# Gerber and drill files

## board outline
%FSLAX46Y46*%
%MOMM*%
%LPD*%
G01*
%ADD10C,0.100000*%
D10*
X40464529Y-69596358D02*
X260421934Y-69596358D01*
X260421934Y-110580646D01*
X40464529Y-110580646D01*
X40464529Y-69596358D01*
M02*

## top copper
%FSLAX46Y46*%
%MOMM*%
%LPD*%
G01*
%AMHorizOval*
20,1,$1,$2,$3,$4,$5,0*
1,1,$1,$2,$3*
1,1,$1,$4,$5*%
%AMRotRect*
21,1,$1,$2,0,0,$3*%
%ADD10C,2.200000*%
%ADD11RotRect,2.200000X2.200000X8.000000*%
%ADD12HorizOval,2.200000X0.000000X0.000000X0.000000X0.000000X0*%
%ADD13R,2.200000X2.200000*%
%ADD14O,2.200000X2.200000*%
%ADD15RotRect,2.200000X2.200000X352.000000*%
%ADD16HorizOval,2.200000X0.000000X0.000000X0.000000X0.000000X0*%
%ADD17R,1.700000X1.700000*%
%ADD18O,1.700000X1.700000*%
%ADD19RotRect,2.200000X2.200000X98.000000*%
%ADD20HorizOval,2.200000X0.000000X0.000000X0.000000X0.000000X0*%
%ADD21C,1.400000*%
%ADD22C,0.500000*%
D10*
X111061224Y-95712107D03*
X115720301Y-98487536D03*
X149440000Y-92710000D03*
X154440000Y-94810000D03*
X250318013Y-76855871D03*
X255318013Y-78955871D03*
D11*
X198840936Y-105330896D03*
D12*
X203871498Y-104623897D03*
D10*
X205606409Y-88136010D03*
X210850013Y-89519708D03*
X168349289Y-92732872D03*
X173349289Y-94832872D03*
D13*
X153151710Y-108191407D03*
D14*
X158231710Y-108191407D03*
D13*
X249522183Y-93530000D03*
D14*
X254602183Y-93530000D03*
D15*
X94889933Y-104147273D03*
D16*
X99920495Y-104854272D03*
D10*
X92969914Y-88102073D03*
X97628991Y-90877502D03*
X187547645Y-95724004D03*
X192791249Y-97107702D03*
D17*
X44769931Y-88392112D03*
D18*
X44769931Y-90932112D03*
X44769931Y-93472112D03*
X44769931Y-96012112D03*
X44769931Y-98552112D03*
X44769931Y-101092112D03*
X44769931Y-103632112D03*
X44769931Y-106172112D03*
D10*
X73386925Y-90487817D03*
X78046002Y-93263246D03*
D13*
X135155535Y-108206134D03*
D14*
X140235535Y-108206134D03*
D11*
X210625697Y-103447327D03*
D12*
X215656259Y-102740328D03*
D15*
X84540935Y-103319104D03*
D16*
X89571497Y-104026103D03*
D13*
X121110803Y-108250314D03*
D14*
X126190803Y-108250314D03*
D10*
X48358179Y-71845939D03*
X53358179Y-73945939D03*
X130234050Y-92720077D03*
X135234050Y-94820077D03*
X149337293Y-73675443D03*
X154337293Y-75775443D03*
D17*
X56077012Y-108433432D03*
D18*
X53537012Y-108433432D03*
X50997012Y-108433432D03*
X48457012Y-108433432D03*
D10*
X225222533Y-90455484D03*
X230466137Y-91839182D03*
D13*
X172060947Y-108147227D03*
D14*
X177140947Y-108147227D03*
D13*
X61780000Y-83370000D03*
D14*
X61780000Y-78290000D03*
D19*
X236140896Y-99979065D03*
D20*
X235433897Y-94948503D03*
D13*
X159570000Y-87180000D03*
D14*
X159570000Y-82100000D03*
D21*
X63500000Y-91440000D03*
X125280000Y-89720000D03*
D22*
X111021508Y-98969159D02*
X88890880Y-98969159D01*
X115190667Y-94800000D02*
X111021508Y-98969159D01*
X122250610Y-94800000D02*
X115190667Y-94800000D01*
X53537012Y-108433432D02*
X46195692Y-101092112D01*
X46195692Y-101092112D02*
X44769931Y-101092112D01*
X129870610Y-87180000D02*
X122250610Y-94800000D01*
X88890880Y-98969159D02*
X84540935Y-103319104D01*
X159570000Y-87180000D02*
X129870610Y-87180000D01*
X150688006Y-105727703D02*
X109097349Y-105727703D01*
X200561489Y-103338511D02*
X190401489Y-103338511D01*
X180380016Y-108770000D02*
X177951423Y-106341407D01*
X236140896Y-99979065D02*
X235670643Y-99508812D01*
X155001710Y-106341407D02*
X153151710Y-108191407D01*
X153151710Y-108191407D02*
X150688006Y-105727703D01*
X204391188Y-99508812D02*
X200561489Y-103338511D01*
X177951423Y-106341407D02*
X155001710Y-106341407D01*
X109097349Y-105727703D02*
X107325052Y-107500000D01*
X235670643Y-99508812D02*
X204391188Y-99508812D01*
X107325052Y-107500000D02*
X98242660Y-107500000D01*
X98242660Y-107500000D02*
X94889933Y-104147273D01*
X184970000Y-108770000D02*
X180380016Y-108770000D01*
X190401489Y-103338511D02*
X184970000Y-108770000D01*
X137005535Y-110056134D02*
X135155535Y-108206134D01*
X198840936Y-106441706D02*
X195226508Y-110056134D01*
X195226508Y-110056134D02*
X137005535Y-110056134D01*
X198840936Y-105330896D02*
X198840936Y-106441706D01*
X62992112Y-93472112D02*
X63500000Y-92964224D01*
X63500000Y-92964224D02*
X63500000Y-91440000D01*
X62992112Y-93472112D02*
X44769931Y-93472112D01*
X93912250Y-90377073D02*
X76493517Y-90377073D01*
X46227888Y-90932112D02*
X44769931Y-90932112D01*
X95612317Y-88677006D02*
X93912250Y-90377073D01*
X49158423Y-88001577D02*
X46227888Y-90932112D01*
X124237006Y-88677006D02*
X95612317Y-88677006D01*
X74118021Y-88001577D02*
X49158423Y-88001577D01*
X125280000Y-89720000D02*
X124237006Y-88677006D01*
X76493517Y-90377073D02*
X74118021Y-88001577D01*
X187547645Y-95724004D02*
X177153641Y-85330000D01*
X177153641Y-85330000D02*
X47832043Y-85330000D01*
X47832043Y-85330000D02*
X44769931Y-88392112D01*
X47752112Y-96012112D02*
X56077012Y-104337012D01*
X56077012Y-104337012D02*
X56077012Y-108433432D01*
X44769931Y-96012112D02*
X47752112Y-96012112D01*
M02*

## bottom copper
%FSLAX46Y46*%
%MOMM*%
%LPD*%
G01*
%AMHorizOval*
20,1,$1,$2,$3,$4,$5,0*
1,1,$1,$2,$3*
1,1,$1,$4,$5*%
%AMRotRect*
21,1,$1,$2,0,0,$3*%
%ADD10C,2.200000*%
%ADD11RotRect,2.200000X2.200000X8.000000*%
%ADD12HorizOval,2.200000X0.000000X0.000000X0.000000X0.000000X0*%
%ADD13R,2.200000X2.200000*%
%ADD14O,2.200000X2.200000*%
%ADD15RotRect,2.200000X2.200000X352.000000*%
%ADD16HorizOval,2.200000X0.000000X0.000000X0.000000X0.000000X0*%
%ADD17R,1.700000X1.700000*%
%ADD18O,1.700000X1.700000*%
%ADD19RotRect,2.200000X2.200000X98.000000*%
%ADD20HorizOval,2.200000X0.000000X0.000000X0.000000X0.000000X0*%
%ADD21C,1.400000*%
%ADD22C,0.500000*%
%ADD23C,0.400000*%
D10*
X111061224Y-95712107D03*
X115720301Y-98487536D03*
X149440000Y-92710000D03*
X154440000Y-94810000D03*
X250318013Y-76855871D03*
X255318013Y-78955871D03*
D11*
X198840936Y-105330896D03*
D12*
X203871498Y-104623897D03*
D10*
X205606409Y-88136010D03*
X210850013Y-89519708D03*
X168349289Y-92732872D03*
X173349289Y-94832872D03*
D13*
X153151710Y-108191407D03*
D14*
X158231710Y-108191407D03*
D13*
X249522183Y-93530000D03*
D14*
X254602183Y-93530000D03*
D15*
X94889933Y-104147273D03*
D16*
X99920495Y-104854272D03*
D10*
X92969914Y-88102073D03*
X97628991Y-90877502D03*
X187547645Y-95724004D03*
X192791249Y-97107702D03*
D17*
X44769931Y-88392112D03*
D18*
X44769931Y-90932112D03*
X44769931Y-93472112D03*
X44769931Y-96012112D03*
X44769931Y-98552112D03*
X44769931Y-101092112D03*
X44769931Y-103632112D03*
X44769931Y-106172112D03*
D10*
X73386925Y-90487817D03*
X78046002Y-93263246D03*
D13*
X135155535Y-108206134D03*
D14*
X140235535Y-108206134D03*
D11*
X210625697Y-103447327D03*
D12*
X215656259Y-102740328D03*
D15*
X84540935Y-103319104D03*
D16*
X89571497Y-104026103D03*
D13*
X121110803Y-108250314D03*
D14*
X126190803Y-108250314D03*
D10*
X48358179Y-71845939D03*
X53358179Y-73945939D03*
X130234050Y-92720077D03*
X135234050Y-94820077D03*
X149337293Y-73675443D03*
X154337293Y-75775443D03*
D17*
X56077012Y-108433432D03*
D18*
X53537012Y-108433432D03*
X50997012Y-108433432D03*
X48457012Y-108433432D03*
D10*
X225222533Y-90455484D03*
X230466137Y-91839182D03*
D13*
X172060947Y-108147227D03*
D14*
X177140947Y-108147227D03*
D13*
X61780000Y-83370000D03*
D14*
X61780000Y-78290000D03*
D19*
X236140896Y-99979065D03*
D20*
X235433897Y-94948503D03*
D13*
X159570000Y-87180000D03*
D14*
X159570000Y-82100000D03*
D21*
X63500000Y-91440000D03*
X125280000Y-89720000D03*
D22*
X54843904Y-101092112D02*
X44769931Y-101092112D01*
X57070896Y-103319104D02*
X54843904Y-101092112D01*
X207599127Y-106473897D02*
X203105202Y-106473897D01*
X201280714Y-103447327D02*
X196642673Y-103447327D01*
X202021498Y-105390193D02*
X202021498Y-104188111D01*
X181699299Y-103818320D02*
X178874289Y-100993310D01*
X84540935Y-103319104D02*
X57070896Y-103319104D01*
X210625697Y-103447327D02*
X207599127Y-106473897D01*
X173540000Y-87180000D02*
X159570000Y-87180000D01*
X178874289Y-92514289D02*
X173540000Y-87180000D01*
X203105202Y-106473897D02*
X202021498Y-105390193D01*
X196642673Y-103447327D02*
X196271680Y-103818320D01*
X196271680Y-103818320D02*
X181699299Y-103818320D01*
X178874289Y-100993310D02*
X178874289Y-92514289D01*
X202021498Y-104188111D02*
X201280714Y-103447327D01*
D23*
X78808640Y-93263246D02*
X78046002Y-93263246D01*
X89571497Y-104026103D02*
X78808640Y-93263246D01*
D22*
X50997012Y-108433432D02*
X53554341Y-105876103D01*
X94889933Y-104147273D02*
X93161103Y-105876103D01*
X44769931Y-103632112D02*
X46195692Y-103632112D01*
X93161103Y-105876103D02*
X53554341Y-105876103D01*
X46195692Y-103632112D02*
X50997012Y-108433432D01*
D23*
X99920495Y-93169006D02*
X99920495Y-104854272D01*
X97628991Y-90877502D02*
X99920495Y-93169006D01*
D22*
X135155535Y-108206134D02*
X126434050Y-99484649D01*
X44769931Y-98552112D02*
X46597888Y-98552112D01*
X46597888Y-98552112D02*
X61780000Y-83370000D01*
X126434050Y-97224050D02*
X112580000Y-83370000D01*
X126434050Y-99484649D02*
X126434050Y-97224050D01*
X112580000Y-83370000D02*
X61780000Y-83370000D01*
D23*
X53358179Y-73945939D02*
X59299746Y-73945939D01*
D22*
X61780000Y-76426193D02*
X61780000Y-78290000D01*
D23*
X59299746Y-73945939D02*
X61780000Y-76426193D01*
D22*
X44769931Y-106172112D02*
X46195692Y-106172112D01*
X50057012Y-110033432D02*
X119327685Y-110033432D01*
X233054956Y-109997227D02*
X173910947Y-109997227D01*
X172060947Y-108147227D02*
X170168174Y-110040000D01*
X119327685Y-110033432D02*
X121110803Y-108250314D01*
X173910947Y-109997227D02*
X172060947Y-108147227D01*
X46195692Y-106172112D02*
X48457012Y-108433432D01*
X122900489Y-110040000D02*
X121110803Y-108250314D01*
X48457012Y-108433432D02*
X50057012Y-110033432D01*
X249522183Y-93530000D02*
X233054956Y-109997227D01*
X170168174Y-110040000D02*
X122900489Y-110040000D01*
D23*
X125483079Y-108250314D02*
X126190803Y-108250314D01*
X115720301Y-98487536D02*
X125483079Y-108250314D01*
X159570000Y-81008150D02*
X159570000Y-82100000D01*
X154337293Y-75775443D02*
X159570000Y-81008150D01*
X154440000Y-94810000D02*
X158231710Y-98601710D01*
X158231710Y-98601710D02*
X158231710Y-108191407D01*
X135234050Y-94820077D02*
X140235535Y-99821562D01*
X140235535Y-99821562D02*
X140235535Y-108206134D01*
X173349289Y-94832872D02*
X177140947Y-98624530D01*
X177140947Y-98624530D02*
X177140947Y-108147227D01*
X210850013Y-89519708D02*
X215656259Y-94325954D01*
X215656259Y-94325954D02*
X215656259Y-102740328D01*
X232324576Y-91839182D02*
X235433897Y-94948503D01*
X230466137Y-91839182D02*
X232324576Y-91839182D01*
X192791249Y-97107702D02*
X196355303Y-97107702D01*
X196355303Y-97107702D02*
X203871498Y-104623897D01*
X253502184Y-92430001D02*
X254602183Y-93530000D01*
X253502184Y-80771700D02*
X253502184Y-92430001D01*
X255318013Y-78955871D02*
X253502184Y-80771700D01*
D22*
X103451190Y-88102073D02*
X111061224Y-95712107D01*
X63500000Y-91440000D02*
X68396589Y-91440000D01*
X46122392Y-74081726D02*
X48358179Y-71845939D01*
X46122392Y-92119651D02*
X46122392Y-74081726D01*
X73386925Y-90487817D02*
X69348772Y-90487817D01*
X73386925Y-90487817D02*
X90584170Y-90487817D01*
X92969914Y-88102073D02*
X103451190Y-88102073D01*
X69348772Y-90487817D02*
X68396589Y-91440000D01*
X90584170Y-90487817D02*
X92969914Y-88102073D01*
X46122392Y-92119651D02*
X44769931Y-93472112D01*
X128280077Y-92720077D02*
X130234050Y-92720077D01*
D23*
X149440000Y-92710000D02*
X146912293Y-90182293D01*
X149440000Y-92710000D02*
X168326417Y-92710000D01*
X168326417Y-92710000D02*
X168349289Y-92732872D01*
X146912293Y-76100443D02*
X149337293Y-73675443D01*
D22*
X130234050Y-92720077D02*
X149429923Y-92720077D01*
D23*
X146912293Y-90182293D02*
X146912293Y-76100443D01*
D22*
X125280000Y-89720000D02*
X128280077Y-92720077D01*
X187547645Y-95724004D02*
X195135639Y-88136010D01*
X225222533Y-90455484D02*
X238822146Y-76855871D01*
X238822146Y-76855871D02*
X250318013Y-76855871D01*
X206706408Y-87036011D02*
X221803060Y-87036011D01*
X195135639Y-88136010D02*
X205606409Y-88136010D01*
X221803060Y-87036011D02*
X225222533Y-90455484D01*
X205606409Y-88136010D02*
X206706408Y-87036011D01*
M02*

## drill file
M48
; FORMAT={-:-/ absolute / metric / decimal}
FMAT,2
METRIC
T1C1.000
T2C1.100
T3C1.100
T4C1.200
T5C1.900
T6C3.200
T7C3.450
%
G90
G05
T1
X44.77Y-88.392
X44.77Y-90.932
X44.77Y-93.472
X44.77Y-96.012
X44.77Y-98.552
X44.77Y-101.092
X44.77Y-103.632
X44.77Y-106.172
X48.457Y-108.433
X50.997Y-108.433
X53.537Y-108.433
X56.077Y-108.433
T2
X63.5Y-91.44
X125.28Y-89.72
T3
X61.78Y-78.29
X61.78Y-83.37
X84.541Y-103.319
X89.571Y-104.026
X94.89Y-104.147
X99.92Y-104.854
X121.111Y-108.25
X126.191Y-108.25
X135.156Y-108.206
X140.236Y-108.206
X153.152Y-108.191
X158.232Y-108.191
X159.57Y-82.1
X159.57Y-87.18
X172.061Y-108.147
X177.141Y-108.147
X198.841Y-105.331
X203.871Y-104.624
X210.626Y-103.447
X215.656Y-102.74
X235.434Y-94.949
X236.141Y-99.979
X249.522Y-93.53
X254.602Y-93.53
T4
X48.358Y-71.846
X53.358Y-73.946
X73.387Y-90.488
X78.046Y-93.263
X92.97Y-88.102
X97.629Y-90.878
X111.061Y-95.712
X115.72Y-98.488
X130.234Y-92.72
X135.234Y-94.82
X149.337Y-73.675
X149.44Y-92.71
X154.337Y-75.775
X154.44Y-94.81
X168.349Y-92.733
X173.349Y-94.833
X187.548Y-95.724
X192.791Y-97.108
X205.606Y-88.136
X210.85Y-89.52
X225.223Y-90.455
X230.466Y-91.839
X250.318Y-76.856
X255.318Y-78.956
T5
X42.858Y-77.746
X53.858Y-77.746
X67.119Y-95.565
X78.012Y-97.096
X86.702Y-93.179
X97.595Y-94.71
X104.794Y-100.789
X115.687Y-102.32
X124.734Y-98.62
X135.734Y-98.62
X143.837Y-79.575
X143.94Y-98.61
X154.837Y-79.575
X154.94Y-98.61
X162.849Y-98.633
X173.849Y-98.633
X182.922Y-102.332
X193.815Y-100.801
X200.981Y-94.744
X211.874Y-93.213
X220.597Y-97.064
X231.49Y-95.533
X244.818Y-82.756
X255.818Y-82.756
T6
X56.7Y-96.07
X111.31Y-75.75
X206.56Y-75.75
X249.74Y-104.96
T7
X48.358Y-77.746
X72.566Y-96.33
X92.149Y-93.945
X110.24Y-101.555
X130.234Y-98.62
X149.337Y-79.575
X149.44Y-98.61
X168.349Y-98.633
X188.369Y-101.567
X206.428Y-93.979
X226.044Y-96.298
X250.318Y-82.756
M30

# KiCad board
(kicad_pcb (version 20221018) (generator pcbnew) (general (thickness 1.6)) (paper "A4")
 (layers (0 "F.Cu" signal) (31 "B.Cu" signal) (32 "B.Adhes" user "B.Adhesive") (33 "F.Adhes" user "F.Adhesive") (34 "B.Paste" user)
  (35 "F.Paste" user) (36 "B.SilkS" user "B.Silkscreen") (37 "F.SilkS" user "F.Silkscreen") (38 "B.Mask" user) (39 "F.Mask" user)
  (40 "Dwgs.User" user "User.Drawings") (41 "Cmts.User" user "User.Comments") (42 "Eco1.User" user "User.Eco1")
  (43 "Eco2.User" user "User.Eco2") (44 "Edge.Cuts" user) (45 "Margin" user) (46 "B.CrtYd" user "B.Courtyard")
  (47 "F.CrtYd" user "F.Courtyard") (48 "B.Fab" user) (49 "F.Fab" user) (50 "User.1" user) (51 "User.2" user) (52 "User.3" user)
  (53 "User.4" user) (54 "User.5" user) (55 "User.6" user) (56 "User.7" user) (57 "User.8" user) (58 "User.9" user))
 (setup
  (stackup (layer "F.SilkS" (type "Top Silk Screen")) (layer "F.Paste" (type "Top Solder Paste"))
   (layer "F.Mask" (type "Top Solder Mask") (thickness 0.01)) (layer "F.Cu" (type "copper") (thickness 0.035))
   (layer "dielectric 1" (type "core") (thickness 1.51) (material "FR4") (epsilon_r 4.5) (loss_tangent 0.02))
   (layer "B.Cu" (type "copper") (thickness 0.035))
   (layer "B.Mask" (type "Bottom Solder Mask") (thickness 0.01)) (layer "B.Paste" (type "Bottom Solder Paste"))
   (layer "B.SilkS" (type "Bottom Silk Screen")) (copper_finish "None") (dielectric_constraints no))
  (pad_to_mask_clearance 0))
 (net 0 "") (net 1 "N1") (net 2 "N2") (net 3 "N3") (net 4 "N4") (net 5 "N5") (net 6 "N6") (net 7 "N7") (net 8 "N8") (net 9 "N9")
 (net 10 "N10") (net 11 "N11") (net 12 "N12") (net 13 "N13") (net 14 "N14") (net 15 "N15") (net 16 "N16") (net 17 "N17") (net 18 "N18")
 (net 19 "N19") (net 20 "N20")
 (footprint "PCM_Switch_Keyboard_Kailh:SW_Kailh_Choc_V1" (layer "F.Cu") (at 110.240103 101.554689 -8)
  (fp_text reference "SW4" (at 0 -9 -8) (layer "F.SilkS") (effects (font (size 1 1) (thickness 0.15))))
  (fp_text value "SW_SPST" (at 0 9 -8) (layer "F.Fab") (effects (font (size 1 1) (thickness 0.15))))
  (pad "" np_thru_hole circle (at -5.5 0 352) (size 1.9 1.9) (drill 1.9) (layers "*.Cu" "*.Mask"))
  (pad "" smd circle (at 0 -5.9 352) (size 1.25 1.25) (layers "F.Mask"))
  (pad "" np_thru_hole circle (at 0 0 352) (size 3.45 3.45) (drill 3.45) (layers "*.Cu" "*.Mask"))
  (pad "" smd circle (at 5 -3.8 352) (size 1.25 1.25) (layers "F.Mask"))
  (pad "" np_thru_hole circle (at 5.5 0 352) (size 1.9 1.9) (drill 1.9) (layers "*.Cu" "*.Mask"))
  (pad "1" thru_hole circle (at 0 -5.9 352) (size 2.2 2.2) (drill 1.2) (layers "*.Cu" "B.Mask") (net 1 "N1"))
  (pad "2" thru_hole circle (at 5 -3.8 352) (size 2.2 2.2) (drill 1.2) (layers "*.Cu" "B.Mask") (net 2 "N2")))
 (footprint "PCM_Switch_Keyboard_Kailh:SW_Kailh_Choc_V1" (layer "F.Cu") (at 149.44 98.61)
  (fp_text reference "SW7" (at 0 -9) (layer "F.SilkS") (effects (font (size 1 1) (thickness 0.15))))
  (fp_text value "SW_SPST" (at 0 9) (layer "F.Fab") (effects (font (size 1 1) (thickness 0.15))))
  (pad "" np_thru_hole circle (at -5.5 0) (size 1.9 1.9) (drill 1.9) (layers "*.Cu" "*.Mask"))
  (pad "" smd circle (at 0 -5.9) (size 1.25 1.25) (layers "F.Mask"))
  (pad "" np_thru_hole circle (at 0 0) (size 3.45 3.45) (drill 3.45) (layers "*.Cu" "*.Mask"))
  (pad "" smd circle (at 5 -3.8) (size 1.25 1.25) (layers "F.Mask"))
  (pad "" np_thru_hole circle (at 5.5 0) (size 1.9 1.9) (drill 1.9) (layers "*.Cu" "*.Mask"))
  (pad "1" thru_hole circle (at 0 -5.9) (size 2.2 2.2) (drill 1.2) (layers "*.Cu" "B.Mask") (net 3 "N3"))
  (pad "2" thru_hole circle (at 5 -3.8) (size 2.2 2.2) (drill 1.2) (layers "*.Cu" "B.Mask") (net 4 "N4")))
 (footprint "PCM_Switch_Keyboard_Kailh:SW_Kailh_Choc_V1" (layer "F.Cu") (at 250.318013 82.755871)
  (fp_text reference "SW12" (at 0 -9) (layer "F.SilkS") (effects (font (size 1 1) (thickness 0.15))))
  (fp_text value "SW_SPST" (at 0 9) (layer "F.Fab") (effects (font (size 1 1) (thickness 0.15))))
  (pad "" np_thru_hole circle (at -5.5 0) (size 1.9 1.9) (drill 1.9) (layers "*.Cu" "*.Mask"))
  (pad "" smd circle (at 0 -5.9) (size 1.25 1.25) (layers "F.Mask"))
  (pad "" np_thru_hole circle (at 0 0) (size 3.45 3.45) (drill 3.45) (layers "*.Cu" "*.Mask"))
  (pad "" smd circle (at 5 -3.8) (size 1.25 1.25) (layers "F.Mask"))
  (pad "" np_thru_hole circle (at 5.5 0) (size 1.9 1.9) (drill 1.9) (layers "*.Cu" "*.Mask"))
  (pad "1" thru_hole circle (at 0 -5.9) (size 2.2 2.2) (drill 1.2) (layers "*.Cu" "B.Mask") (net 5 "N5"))
  (pad "2" thru_hole circle (at 5 -3.8) (size 2.2 2.2) (drill 1.2) (layers "*.Cu" "B.Mask") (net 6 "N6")))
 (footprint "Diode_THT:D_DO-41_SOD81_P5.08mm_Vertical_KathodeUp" (layer "F.Cu") (at 198.840936 105.330896 8)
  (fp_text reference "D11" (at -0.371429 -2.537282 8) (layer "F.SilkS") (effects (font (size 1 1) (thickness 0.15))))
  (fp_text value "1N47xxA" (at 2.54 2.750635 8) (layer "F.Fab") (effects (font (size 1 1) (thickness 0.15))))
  (pad "1" thru_hole rect (at 0 0 8) (size 2.2 2.2) (drill 1.1) (layers "*.Cu" "*.Mask") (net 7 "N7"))
  (pad "2" thru_hole oval (at 5.08 0 8) (size 2.2 2.2) (drill 1.1) (layers "*.Cu" "*.Mask") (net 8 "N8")))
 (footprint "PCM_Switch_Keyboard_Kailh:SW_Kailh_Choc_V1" (layer "F.Cu") (at 206.42753 93.978592 8)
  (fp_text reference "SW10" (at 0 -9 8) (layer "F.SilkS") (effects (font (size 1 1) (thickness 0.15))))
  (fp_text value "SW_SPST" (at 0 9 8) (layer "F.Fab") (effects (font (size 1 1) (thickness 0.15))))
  (pad "" np_thru_hole circle (at -5.5 0 8) (size 1.9 1.9) (drill 1.9) (layers "*.Cu" "*.Mask"))
  (pad "" smd circle (at 0 -5.9 8) (size 1.25 1.25) (layers "F.Mask"))
  (pad "" np_thru_hole circle (at 0 0 8) (size 3.45 3.45) (drill 3.45) (layers "*.Cu" "*.Mask"))
  (pad "" smd circle (at 5 -3.8 8) (size 1.25 1.25) (layers "F.Mask"))
  (pad "" np_thru_hole circle (at 5.5 0 8) (size 1.9 1.9) (drill 1.9) (layers "*.Cu" "*.Mask"))
  (pad "1" thru_hole circle (at 0 -5.9 8) (size 2.2 2.2) (drill 1.2) (layers "*.Cu" "B.Mask") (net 5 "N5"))
  (pad "2" thru_hole circle (at 5 -3.8 8) (size 2.2 2.2) (drill 1.2) (layers "*.Cu" "B.Mask") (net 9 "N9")))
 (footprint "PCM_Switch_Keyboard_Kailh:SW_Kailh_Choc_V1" (layer "F.Cu") (at 168.349289 98.632872)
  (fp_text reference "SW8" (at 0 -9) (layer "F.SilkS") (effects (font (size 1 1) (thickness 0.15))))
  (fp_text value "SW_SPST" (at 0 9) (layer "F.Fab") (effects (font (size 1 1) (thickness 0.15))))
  (pad "" np_thru_hole circle (at -5.5 0) (size 1.9 1.9) (drill 1.9) (layers "*.Cu" "*.Mask"))
  (pad "" smd circle (at 0 -5.9) (size 1.25 1.25) (layers "F.Mask"))
  (pad "" np_thru_hole circle (at 0 0) (size 3.45 3.45) (drill 3.45) (layers "*.Cu" "*.Mask"))
  (pad "" smd circle (at 5 -3.8) (size 1.25 1.25) (layers "F.Mask"))
  (pad "" np_thru_hole circle (at 5.5 0) (size 1.9 1.9) (drill 1.9) (layers "*.Cu" "*.Mask"))
  (pad "1" thru_hole circle (at 0 -5.9) (size 2.2 2.2) (drill 1.2) (layers "*.Cu" "B.Mask") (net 3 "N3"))
  (pad "2" thru_hole circle (at 5 -3.8) (size 2.2 2.2) (drill 1.2) (layers "*.Cu" "B.Mask") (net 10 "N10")))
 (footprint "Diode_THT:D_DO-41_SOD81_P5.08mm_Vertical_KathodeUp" (layer "F.Cu") (at 153.15171 108.191407)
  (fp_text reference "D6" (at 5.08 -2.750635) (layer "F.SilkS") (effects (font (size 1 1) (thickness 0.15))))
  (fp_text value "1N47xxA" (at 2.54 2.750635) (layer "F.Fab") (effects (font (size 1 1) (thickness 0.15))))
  (pad "1" thru_hole rect (at 0 0) (size 2.2 2.2) (drill 1.1) (layers "*.Cu" "*.Mask") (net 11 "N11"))
  (pad "2" thru_hole oval (at 5.08 0) (size 2.2 2.2) (drill 1.1) (layers "*.Cu" "*.Mask") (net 4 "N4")))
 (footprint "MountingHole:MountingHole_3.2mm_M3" (layer "F.Cu") (at 249.74 104.96)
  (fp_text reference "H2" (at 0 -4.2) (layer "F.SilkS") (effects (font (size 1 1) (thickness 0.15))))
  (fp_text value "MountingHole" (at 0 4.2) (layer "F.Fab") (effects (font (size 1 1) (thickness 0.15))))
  (pad "" np_thru_hole circle (at 0 0) (size 3.2 3.2) (drill 3.2) (layers "*.Cu" "*.Mask")))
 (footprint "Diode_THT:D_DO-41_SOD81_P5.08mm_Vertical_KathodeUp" (layer "F.Cu") (at 249.522183 93.53)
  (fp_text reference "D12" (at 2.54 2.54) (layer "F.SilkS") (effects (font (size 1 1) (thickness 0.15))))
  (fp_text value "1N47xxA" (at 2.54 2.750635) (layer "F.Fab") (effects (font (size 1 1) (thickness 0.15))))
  (pad "1" thru_hole rect (at 0 0) (size 2.2 2.2) (drill 1.1) (layers "*.Cu" "*.Mask") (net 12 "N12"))
  (pad "2" thru_hole oval (at 5.08 0) (size 2.2 2.2) (drill 1.1) (layers "*.Cu" "*.Mask") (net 6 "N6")))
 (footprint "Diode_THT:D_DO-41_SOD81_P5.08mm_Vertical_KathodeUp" (layer "F.Cu") (at 94.889933 104.147273 -8)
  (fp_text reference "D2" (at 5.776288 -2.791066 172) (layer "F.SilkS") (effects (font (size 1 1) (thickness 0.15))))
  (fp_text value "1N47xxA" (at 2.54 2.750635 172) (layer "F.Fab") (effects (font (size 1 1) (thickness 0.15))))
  (pad "1" thru_hole rect (at 0 0 352) (size 2.2 2.2) (drill 1.1) (layers "*.Cu" "*.Mask") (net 11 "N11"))
  (pad "2" thru_hole oval (at 5.08 0 352) (size 2.2 2.2) (drill 1.1) (layers "*.Cu" "*.Mask") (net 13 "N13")))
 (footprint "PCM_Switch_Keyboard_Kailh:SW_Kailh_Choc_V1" (layer "F.Cu") (at 92.148793 93.944655 -8)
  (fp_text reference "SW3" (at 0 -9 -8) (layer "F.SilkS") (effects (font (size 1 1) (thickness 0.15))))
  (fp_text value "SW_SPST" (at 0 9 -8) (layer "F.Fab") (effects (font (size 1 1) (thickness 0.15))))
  (pad "" np_thru_hole circle (at -5.5 0 352) (size 1.9 1.9) (drill 1.9) (layers "*.Cu" "*.Mask"))
  (pad "" smd circle (at 0 -5.9 352) (size 1.25 1.25) (layers "F.Mask"))
  (pad "" np_thru_hole circle (at 0 0 352) (size 3.45 3.45) (drill 3.45) (layers "*.Cu" "*.Mask"))
  (pad "" smd circle (at 5 -3.8 352) (size 1.25 1.25) (layers "F.Mask"))
  (pad "" np_thru_hole circle (at 5.5 0 352) (size 1.9 1.9) (drill 1.9) (layers "*.Cu" "*.Mask"))
  (pad "1" thru_hole circle (at 0 -5.9 352) (size 2.2 2.2) (drill 1.2) (layers "*.Cu" "B.Mask") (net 1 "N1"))
  (pad "2" thru_hole circle (at 5 -3.8 352) (size 2.2 2.2) (drill 1.2) (layers "*.Cu" "B.Mask") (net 13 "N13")))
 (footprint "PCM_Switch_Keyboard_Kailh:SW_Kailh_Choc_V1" (layer "F.Cu") (at 188.368766 101.566586 8)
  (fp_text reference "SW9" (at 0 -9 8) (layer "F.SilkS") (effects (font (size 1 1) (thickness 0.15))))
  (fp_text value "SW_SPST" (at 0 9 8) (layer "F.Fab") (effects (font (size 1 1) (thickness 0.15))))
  (pad "" np_thru_hole circle (at -5.5 0 8) (size 1.9 1.9) (drill 1.9) (layers "*.Cu" "*.Mask"))
  (pad "" smd circle (at 0 -5.9 8) (size 1.25 1.25) (layers "F.Mask"))
  (pad "" np_thru_hole circle (at 0 0 8) (size 3.45 3.45) (drill 3.45) (layers "*.Cu" "*.Mask"))
  (pad "" smd circle (at 5 -3.8 8) (size 1.25 1.25) (layers "F.Mask"))
  (pad "" np_thru_hole circle (at 5.5 0 8) (size 1.9 1.9) (drill 1.9) (layers "*.Cu" "*.Mask"))
  (pad "1" thru_hole circle (at 0 -5.9 8) (size 2.2 2.2) (drill 1.2) (layers "*.Cu" "B.Mask") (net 5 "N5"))
  (pad "2" thru_hole circle (at 5 -3.8 8) (size 2.2 2.2) (drill 1.2) (layers "*.Cu" "B.Mask") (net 8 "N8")))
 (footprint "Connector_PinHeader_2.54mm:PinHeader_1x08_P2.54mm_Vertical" (layer "F.Cu") (at 44.769931 88.392112)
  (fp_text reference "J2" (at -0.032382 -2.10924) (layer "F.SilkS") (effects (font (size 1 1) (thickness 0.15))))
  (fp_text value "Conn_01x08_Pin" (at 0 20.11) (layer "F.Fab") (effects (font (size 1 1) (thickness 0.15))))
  (pad "1" thru_hole rect (at 0 0) (size 1.7 1.7) (drill 1) (layers "*.Cu" "*.Mask") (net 5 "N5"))
  (pad "2" thru_hole oval (at 0 2.54) (size 1.7 1.7) (drill 1) (layers "*.Cu" "*.Mask") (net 3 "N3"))
  (pad "3" thru_hole oval (at 0 5.08) (size 1.7 1.7) (drill 1) (layers "*.Cu" "*.Mask") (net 1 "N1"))
  (pad "4" thru_hole oval (at 0 7.62) (size 1.7 1.7) (drill 1) (layers "*.Cu" "*.Mask") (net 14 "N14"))
  (pad "5" thru_hole oval (at 0 10.16) (size 1.7 1.7) (drill 1) (layers "*.Cu" "*.Mask") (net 7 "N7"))
  (pad "6" thru_hole oval (at 0 12.7) (size 1.7 1.7) (drill 1) (layers "*.Cu" "*.Mask") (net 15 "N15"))
  (pad "7" thru_hole oval (at 0 15.24) (size 1.7 1.7) (drill 1) (layers "*.Cu" "*.Mask") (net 11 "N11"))
  (pad "8" thru_hole oval (at 0 17.78) (size 1.7 1.7) (drill 1) (layers "*.Cu" "*.Mask") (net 12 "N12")))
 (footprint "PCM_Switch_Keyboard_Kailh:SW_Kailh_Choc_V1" (layer "F.Cu") (at 72.565804 96.330399 -8)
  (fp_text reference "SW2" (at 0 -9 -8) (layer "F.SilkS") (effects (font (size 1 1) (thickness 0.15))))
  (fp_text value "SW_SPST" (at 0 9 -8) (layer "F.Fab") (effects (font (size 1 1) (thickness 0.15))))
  (pad "" np_thru_hole circle (at -5.5 0 352) (size 1.9 1.9) (drill 1.9) (layers "*.Cu" "*.Mask"))
  (pad "" smd circle (at 0 -5.9 352) (size 1.25 1.25) (layers "F.Mask"))
  (pad "" np_thru_hole circle (at 0 0 352) (size 3.45 3.45) (drill 3.45) (layers "*.Cu" "*.Mask"))
  (pad "" smd circle (at 5 -3.8 352) (size 1.25 1.25) (layers "F.Mask"))
  (pad "" np_thru_hole circle (at 5.5 0 352) (size 1.9 1.9) (drill 1.9) (layers "*.Cu" "*.Mask"))
  (pad "1" thru_hole circle (at 0 -5.9 352) (size 2.2 2.2) (drill 1.2) (layers "*.Cu" "B.Mask") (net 1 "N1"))
  (pad "2" thru_hole circle (at 5 -3.8 352) (size 2.2 2.2) (drill 1.2) (layers "*.Cu" "B.Mask") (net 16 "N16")))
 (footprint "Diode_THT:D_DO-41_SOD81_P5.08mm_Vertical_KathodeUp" (layer "F.Cu") (at 135.155535 108.206134)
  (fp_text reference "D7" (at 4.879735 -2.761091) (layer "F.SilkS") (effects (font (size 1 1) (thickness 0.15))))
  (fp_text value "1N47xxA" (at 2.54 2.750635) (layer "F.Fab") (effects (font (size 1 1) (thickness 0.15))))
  (pad "1" thru_hole rect (at 0 0) (size 2.2 2.2) (drill 1.1) (layers "*.Cu" "*.Mask") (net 7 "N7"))
  (pad "2" thru_hole oval (at 5.08 0) (size 2.2 2.2) (drill 1.1) (layers "*.Cu" "*.Mask") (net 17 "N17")))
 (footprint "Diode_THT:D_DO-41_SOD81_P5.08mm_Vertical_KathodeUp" (layer "F.Cu") (at 210.625697 103.447327 8)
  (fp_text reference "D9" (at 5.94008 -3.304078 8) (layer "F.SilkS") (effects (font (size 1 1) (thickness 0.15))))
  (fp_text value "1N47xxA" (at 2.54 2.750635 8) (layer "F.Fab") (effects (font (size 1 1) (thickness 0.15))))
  (pad "1" thru_hole rect (at 0 0 8) (size 2.2 2.2) (drill 1.1) (layers "*.Cu" "*.Mask") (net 15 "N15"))
  (pad "2" thru_hole oval (at 5.08 0 8) (size 2.2 2.2) (drill 1.1) (layers "*.Cu" "*.Mask") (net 9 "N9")))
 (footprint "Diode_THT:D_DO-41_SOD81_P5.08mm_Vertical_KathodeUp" (layer "F.Cu") (at 84.540935 103.319104 -8)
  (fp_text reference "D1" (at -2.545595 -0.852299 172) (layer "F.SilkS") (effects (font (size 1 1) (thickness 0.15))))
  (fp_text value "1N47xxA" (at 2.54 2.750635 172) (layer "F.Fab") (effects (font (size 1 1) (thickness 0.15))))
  (pad "1" thru_hole rect (at 0 0 352) (size 2.2 2.2) (drill 1.1) (layers "*.Cu" "*.Mask") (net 15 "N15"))
  (pad "2" thru_hole oval (at 5.08 0 352) (size 2.2 2.2) (drill 1.1) (layers "*.Cu" "*.Mask") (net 16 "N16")))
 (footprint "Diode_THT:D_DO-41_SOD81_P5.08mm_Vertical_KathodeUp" (layer "F.Cu") (at 121.110803 108.250314)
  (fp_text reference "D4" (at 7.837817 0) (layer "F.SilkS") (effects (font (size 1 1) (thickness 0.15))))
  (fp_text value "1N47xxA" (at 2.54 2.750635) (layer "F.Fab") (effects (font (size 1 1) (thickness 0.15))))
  (pad "1" thru_hole rect (at 0 0) (size 2.2 2.2) (drill 1.1) (layers "*.Cu" "*.Mask") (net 12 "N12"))
  (pad "2" thru_hole oval (at 5.08 0) (size 2.2 2.2) (drill 1.1) (layers "*.Cu" "*.Mask") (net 2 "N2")))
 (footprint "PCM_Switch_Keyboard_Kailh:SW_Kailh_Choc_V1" (layer "F.Cu") (at 48.358179 77.745939)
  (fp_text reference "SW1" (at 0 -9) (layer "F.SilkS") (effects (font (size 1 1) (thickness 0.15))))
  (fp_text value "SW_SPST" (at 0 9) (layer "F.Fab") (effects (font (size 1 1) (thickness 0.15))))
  (pad "" np_thru_hole circle (at -5.5 0) (size 1.9 1.9) (drill 1.9) (layers "*.Cu" "*.Mask"))
  (pad "" smd circle (at 0 -5.9) (size 1.25 1.25) (layers "F.Mask"))
  (pad "" np_thru_hole circle (at 0 0) (size 3.45 3.45) (drill 3.45) (layers "*.Cu" "*.Mask"))
  (pad "" smd circle (at 5 -3.8) (size 1.25 1.25) (layers "F.Mask"))
  (pad "" np_thru_hole circle (at 5.5 0) (size 1.9 1.9) (drill 1.9) (layers "*.Cu" "*.Mask"))
  (pad "1" thru_hole circle (at 0 -5.9) (size 2.2 2.2) (drill 1.2) (layers "*.Cu" "B.Mask") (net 1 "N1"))
  (pad "2" thru_hole circle (at 5 -3.8) (size 2.2 2.2) (drill 1.2) (layers "*.Cu" "B.Mask") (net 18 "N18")))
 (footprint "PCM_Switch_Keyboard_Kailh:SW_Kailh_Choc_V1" (layer "F.Cu") (at 130.23405 98.620077)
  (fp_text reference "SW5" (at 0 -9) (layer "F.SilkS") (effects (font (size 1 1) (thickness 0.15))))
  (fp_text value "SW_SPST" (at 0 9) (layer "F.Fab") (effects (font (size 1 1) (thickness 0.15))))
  (pad "" np_thru_hole circle (at -5.5 0) (size 1.9 1.9) (drill 1.9) (layers "*.Cu" "*.Mask"))
  (pad "" smd circle (at 0 -5.9) (size 1.25 1.25) (layers "F.Mask"))
  (pad "" np_thru_hole circle (at 0 0) (size 3.45 3.45) (drill 3.45) (layers "*.Cu" "*.Mask"))
  (pad "" smd circle (at 5 -3.8) (size 1.25 1.25) (layers "F.Mask"))
  (pad "" np_thru_hole circle (at 5.5 0) (size 1.9 1.9) (drill 1.9) (layers "*.Cu" "*.Mask"))
  (pad "1" thru_hole circle (at 0 -5.9) (size 2.2 2.2) (drill 1.2) (layers "*.Cu" "B.Mask") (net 3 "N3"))
  (pad "2" thru_hole circle (at 5 -3.8) (size 2.2 2.2) (drill 1.2) (layers "*.Cu" "B.Mask") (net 17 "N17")))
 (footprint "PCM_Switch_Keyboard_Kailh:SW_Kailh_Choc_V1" (layer "F.Cu") (at 149.337293 79.575443)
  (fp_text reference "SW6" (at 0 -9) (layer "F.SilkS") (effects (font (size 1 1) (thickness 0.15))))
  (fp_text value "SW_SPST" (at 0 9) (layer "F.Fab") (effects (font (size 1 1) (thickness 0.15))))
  (pad "" np_thru_hole circle (at -5.5 0) (size 1.9 1.9) (drill 1.9) (layers "*.Cu" "*.Mask"))
  (pad "" smd circle (at 0 -5.9) (size 1.25 1.25) (layers "F.Mask"))
  (pad "" np_thru_hole circle (at 0 0) (size 3.45 3.45) (drill 3.45) (layers "*.Cu" "*.Mask"))
  (pad "" smd circle (at 5 -3.8) (size 1.25 1.25) (layers "F.Mask"))
  (pad "" np_thru_hole circle (at 5.5 0) (size 1.9 1.9) (drill 1.9) (layers "*.Cu" "*.Mask"))
  (pad "1" thru_hole circle (at 0 -5.9) (size 2.2 2.2) (drill 1.2) (layers "*.Cu" "B.Mask") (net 3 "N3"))
  (pad "2" thru_hole circle (at 5 -3.8) (size 2.2 2.2) (drill 1.2) (layers "*.Cu" "B.Mask") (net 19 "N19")))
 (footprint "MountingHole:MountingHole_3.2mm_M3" (layer "F.Cu") (at 111.31 75.75)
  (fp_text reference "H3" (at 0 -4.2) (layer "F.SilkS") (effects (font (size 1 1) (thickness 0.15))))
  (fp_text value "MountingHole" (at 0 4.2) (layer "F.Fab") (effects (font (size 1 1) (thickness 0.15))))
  (pad "" np_thru_hole circle (at 0 0) (size 3.2 3.2) (drill 3.2) (layers "*.Cu" "*.Mask")))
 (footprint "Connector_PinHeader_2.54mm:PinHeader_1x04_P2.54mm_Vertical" (layer "F.Cu") (at 56.077012 108.433432 -90)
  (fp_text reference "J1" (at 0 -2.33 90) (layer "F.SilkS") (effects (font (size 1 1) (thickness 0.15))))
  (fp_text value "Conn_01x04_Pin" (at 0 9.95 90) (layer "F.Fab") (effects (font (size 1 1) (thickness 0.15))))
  (pad "1" thru_hole rect (at 0 0 270) (size 1.7 1.7) (drill 1) (layers "*.Cu" "*.Mask") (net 14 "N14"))
  (pad "2" thru_hole oval (at 0 2.54 270) (size 1.7 1.7) (drill 1) (layers "*.Cu" "*.Mask") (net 15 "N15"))
  (pad "3" thru_hole oval (at 0 5.08 270) (size 1.7 1.7) (drill 1) (layers "*.Cu" "*.Mask") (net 11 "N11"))
  (pad "4" thru_hole oval (at 0 7.62 270) (size 1.7 1.7) (drill 1) (layers "*.Cu" "*.Mask") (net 12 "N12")))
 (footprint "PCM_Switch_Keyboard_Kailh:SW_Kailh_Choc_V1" (layer "F.Cu") (at 226.043654 96.298066 8)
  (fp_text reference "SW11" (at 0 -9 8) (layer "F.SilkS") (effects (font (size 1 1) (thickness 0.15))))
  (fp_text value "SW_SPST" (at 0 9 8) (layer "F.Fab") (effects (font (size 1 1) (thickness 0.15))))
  (pad "" np_thru_hole circle (at -5.5 0 8) (size 1.9 1.9) (drill 1.9) (layers "*.Cu" "*.Mask"))
  (pad "" smd circle (at 0 -5.9 8) (size 1.25 1.25) (layers "F.Mask"))
  (pad "" np_thru_hole circle (at 0 0 8) (size 3.45 3.45) (drill 3.45) (layers "*.Cu" "*.Mask"))
  (pad "" smd circle (at 5 -3.8 8) (size 1.25 1.25) (layers "F.Mask"))
  (pad "" np_thru_hole circle (at 5.5 0 8) (size 1.9 1.9) (drill 1.9) (layers "*.Cu" "*.Mask"))
  (pad "1" thru_hole circle (at 0 -5.9 8) (size 2.2 2.2) (drill 1.2) (layers "*.Cu" "B.Mask") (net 5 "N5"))
  (pad "2" thru_hole circle (at 5 -3.8 8) (size 2.2 2.2) (drill 1.2) (layers "*.Cu" "B.Mask") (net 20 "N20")))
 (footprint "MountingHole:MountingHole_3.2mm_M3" (layer "F.Cu") (at 206.56 75.75)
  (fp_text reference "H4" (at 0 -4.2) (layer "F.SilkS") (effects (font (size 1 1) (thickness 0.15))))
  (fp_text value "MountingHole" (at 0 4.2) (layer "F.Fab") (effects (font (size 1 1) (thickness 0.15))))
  (pad "" np_thru_hole circle (at 0 0) (size 3.2 3.2) (drill 3.2) (layers "*.Cu" "*.Mask")))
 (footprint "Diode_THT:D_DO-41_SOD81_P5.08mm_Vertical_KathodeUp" (layer "F.Cu") (at 172.060947 108.147227)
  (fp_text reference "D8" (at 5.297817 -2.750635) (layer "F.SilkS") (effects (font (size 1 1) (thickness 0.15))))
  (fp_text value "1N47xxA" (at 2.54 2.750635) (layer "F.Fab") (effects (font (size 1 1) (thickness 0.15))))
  (pad "1" thru_hole rect (at 0 0) (size 2.2 2.2) (drill 1.1) (layers "*.Cu" "*.Mask") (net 12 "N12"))
  (pad "2" thru_hole oval (at 5.08 0) (size 2.2 2.2) (drill 1.1) (layers "*.Cu" "*.Mask") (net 10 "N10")))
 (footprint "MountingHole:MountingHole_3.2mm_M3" (layer "F.Cu") (at 56.7 96.07)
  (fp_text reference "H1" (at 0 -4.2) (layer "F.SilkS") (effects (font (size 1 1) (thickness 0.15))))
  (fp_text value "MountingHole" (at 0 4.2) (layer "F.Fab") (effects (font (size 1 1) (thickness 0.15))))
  (pad "" np_thru_hole circle (at 0 0) (size 3.2 3.2) (drill 3.2) (layers "*.Cu" "*.Mask")))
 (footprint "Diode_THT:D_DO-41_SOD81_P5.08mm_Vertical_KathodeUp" (layer "F.Cu") (at 61.78 83.37 90)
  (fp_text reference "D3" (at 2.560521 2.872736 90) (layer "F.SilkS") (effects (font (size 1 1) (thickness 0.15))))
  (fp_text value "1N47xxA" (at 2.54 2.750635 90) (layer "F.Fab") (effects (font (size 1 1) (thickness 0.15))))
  (pad "1" thru_hole rect (at 0 0 90) (size 2.2 2.2) (drill 1.1) (layers "*.Cu" "*.Mask") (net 7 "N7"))
  (pad "2" thru_hole oval (at 5.08 0 90) (size 2.2 2.2) (drill 1.1) (layers "*.Cu" "*.Mask") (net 18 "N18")))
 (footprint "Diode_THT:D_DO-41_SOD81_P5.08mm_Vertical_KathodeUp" (layer "F.Cu") (at 236.140896 99.979065 98)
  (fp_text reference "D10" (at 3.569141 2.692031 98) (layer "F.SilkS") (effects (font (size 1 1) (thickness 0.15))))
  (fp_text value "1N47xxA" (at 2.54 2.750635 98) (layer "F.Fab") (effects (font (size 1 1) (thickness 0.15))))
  (pad "1" thru_hole rect (at 0 0 98) (size 2.2 2.2) (drill 1.1) (layers "*.Cu" "*.Mask") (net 11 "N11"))
  (pad "2" thru_hole oval (at 5.08 0 98) (size 2.2 2.2) (drill 1.1) (layers "*.Cu" "*.Mask") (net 20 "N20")))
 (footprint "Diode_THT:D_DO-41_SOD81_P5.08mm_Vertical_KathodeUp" (layer "F.Cu") (at 159.57 87.18 90)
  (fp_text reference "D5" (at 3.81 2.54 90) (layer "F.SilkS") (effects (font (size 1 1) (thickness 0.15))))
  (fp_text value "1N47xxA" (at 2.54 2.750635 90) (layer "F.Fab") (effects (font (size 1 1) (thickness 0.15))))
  (pad "1" thru_hole rect (at 0 0 90) (size 2.2 2.2) (drill 1.1) (layers "*.Cu" "*.Mask") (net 15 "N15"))
  (pad "2" thru_hole oval (at 5.08 0 90) (size 2.2 2.2) (drill 1.1) (layers "*.Cu" "*.Mask") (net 19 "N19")))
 (gr_rect (start 40.464529 69.596358) (end 260.421934 110.580646) (stroke (width 0.1) (type default)) (fill none) (layer "Edge.Cuts"))
 (segment (start 111.021508 98.969159) (end 88.89088 98.969159) (width 0.5) (layer "F.Cu") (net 15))
 (segment (start 115.190667 94.8) (end 111.021508 98.969159) (width 0.5) (layer "F.Cu") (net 15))
 (segment (start 122.25061 94.8) (end 115.190667 94.8) (width 0.5) (layer "F.Cu") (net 15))
 (segment (start 53.537012 108.433432) (end 46.195692 101.092112) (width 0.5) (layer "F.Cu") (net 15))
 (segment (start 46.195692 101.092112) (end 44.769931 101.092112) (width 0.5) (layer "F.Cu") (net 15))
 (segment (start 129.87061 87.18) (end 122.25061 94.8) (width 0.5) (layer "F.Cu") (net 15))
 (segment (start 88.89088 98.969159) (end 84.540935 103.319104) (width 0.5) (layer "F.Cu") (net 15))
 (segment (start 159.57 87.18) (end 129.87061 87.18) (width 0.5) (layer "F.Cu") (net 15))
 (segment (start 54.843904 101.092112) (end 44.769931 101.092112) (width 0.5) (layer "B.Cu") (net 15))
 (segment (start 57.070896 103.319104) (end 54.843904 101.092112) (width 0.5) (layer "B.Cu") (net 15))
 (segment (start 207.599127 106.473897) (end 203.105202 106.473897) (width 0.5) (layer "B.Cu") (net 15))
 (segment (start 201.280714 103.447327) (end 196.642673 103.447327) (width 0.5) (layer "B.Cu") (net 15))
 (segment (start 202.021498 105.390193) (end 202.021498 104.188111) (width 0.5) (layer "B.Cu") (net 15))
 (segment (start 181.699299 103.81832) (end 178.874289 100.99331) (width 0.5) (layer "B.Cu") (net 15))
 (segment (start 84.540935 103.319104) (end 57.070896 103.319104) (width 0.5) (layer "B.Cu") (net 15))
 (segment (start 210.625697 103.447327) (end 207.599127 106.473897) (width 0.5) (layer "B.Cu") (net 15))
 (segment (start 173.54 87.18) (end 159.57 87.18) (width 0.5) (layer "B.Cu") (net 15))
 (segment (start 178.874289 92.514289) (end 173.54 87.18) (width 0.5) (layer "B.Cu") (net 15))
 (segment (start 203.105202 106.473897) (end 202.021498 105.390193) (width 0.5) (layer "B.Cu") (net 15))
 (segment (start 196.642673 103.447327) (end 196.27168 103.81832) (width 0.5) (layer "B.Cu") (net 15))
 (segment (start 196.27168 103.81832) (end 181.699299 103.81832) (width 0.5) (layer "B.Cu") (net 15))
 (segment (start 178.874289 100.99331) (end 178.874289 92.514289) (width 0.5) (layer "B.Cu") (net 15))
 (segment (start 202.021498 104.188111) (end 201.280714 103.447327) (width 0.5) (layer "B.Cu") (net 15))
 (segment (start 78.80864 93.263246) (end 78.046002 93.263246) (width 0.4) (layer "B.Cu") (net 16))
 (segment (start 89.571497 104.026103) (end 78.80864 93.263246) (width 0.4) (layer "B.Cu") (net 16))
 (segment (start 150.688006 105.727703) (end 109.097349 105.727703) (width 0.5) (layer "F.Cu") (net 11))
 (segment (start 200.561489 103.338511) (end 190.401489 103.338511) (width 0.5) (layer "F.Cu") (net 11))
 (segment (start 180.380016 108.77) (end 177.951423 106.341407) (width 0.5) (layer "F.Cu") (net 11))
 (segment (start 236.140896 99.979065) (end 235.670643 99.508812) (width 0.5) (layer "F.Cu") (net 11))
 (segment (start 155.00171 106.341407) (end 153.15171 108.191407) (width 0.5) (layer "F.Cu") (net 11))
 (segment (start 153.15171 108.191407) (end 150.688006 105.727703) (width 0.5) (layer "F.Cu") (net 11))
 (segment (start 204.391188 99.508812) (end 200.561489 103.338511) (width 0.5) (layer "F.Cu") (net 11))
 (segment (start 177.951423 106.341407) (end 155.00171 106.341407) (width 0.5) (layer "F.Cu") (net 11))
 (segment (start 109.097349 105.727703) (end 107.325052 107.5) (width 0.5) (layer "F.Cu") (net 11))
 (segment (start 235.670643 99.508812) (end 204.391188 99.508812) (width 0.5) (layer "F.Cu") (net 11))
 (segment (start 107.325052 107.5) (end 98.24266 107.5) (width 0.5) (layer "F.Cu") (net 11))
 (segment (start 98.24266 107.5) (end 94.889933 104.147273) (width 0.5) (layer "F.Cu") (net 11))
 (segment (start 184.97 108.77) (end 180.380016 108.77) (width 0.5) (layer "F.Cu") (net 11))
 (segment (start 190.401489 103.338511) (end 184.97 108.77) (width 0.5) (layer "F.Cu") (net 11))
 (segment (start 50.997012 108.433432) (end 53.554341 105.876103) (width 0.5) (layer "B.Cu") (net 11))
 (segment (start 94.889933 104.147273) (end 93.161103 105.876103) (width 0.5) (layer "B.Cu") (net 11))
 (segment (start 44.769931 103.632112) (end 46.195692 103.632112) (width 0.5) (layer "B.Cu") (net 11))
 (segment (start 93.161103 105.876103) (end 53.554341 105.876103) (width 0.5) (layer "B.Cu") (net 11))
 (segment (start 46.195692 103.632112) (end 50.997012 108.433432) (width 0.5) (layer "B.Cu") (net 11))
 (segment (start 99.920495 93.169006) (end 99.920495 104.854272) (width 0.4) (layer "B.Cu") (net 13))
 (segment (start 97.628991 90.877502) (end 99.920495 93.169006) (width 0.4) (layer "B.Cu") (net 13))
 (segment (start 137.005535 110.056134) (end 135.155535 108.206134) (width 0.5) (layer "F.Cu") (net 7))
 (segment (start 198.840936 106.441706) (end 195.226508 110.056134) (width 0.5) (layer "F.Cu") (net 7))
 (segment (start 195.226508 110.056134) (end 137.005535 110.056134) (width 0.5) (layer "F.Cu") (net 7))
 (segment (start 198.840936 105.330896) (end 198.840936 106.441706) (width 0.5) (layer "F.Cu") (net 7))
 (segment (start 135.155535 108.206134) (end 126.43405 99.484649) (width 0.5) (layer "B.Cu") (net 7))
 (segment (start 44.769931 98.552112) (end 46.597888 98.552112) (width 0.5) (layer "B.Cu") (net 7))
 (segment (start 46.597888 98.552112) (end 61.78 83.37) (width 0.5) (layer "B.Cu") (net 7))
 (segment (start 126.43405 97.22405) (end 112.58 83.37) (width 0.5) (layer "B.Cu") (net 7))
 (segment (start 126.43405 99.484649) (end 126.43405 97.22405) (width 0.5) (layer "B.Cu") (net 7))
 (segment (start 112.58 83.37) (end 61.78 83.37) (width 0.5) (layer "B.Cu") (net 7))
 (segment (start 53.358179 73.945939) (end 59.299746 73.945939) (width 0.4) (layer "B.Cu") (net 18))
 (segment (start 61.78 76.426193) (end 61.78 78.29) (width 0.5) (layer "B.Cu") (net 18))
 (segment (start 59.299746 73.945939) (end 61.78 76.426193) (width 0.4) (layer "B.Cu") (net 18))
 (segment (start 44.769931 106.172112) (end 46.195692 106.172112) (width 0.5) (layer "B.Cu") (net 12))
 (segment (start 50.057012 110.033432) (end 119.327685 110.033432) (width 0.5) (layer "B.Cu") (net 12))
 (segment (start 233.054956 109.997227) (end 173.910947 109.997227) (width 0.5) (layer "B.Cu") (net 12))
 (segment (start 172.060947 108.147227) (end 170.168174 110.04) (width 0.5) (layer "B.Cu") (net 12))
 (segment (start 119.327685 110.033432) (end 121.110803 108.250314) (width 0.5) (layer "B.Cu") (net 12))
 (segment (start 173.910947 109.997227) (end 172.060947 108.147227) (width 0.5) (layer "B.Cu") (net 12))
 (segment (start 46.195692 106.172112) (end 48.457012 108.433432) (width 0.5) (layer "B.Cu") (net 12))
 (segment (start 122.900489 110.04) (end 121.110803 108.250314) (width 0.5) (layer "B.Cu") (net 12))
 (segment (start 48.457012 108.433432) (end 50.057012 110.033432) (width 0.5) (layer "B.Cu") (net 12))
 (segment (start 249.522183 93.53) (end 233.054956 109.997227) (width 0.5) (layer "B.Cu") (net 12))
 (segment (start 170.168174 110.04) (end 122.900489 110.04) (width 0.5) (layer "B.Cu") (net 12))
 (segment (start 125.483079 108.250314) (end 126.190803 108.250314) (width 0.4) (layer "B.Cu") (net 2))
 (segment (start 115.720301 98.487536) (end 125.483079 108.250314) (width 0.4) (layer "B.Cu") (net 2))
 (segment (start 159.57 81.00815) (end 159.57 82.1) (width 0.4) (layer "B.Cu") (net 19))
 (segment (start 154.337293 75.775443) (end 159.57 81.00815) (width 0.4) (layer "B.Cu") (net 19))
 (segment (start 154.44 94.81) (end 158.23171 98.60171) (width 0.4) (layer "B.Cu") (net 4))
 (segment (start 158.23171 98.60171) (end 158.23171 108.191407) (width 0.4) (layer "B.Cu") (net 4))
 (segment (start 135.23405 94.820077) (end 140.235535 99.821562) (width 0.4) (layer "B.Cu") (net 17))
 (segment (start 140.235535 99.821562) (end 140.235535 108.206134) (width 0.4) (layer "B.Cu") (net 17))
 (segment (start 173.349289 94.832872) (end 177.140947 98.62453) (width 0.4) (layer "B.Cu") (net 10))
 (segment (start 177.140947 98.62453) (end 177.140947 108.147227) (width 0.4) (layer "B.Cu") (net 10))
 (segment (start 210.850013 89.519708) (end 215.656259 94.325954) (width 0.4) (layer "B.Cu") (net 9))
 (segment (start 215.656259 94.325954) (end 215.656259 102.740328) (width 0.4) (layer "B.Cu") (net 9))
 (segment (start 232.324576 91.839182) (end 235.433897 94.948503) (width 0.4) (layer "B.Cu") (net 20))
 (segment (start 230.466137 91.839182) (end 232.324576 91.839182) (width 0.4) (layer "B.Cu") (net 20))
 (segment (start 192.791249 97.107702) (end 196.355303 97.107702) (width 0.4) (layer "B.Cu") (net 8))
 (segment (start 196.355303 97.107702) (end 203.871498 104.623897) (width 0.4) (layer "B.Cu") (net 8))
 (segment (start 253.502184 92.430001) (end 254.602183 93.53) (width 0.4) (layer "B.Cu") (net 6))
 (segment (start 253.502184 80.7717) (end 253.502184 92.430001) (width 0.4) (layer "B.Cu") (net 6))
 (segment (start 255.318013 78.955871) (end 253.502184 80.7717) (width 0.4) (layer "B.Cu") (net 6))
 (segment (start 62.992112 93.472112) (end 63.5 92.964224) (width 0.5) (layer "F.Cu") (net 1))
 (segment (start 63.5 92.964224) (end 63.5 91.44) (width 0.5) (layer "F.Cu") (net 1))
 (segment (start 62.992112 93.472112) (end 44.769931 93.472112) (width 0.5) (layer "F.Cu") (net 1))
 (via (at 63.5 91.44) (size 1.4) (drill 1.1) (layers "F.Cu" "B.Cu") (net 1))
 (segment (start 103.45119 88.102073) (end 111.061224 95.712107) (width 0.5) (layer "B.Cu") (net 1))
 (segment (start 63.5 91.44) (end 68.396589 91.44) (width 0.5) (layer "B.Cu") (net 1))
 (segment (start 46.122392 74.081726) (end 48.358179 71.845939) (width 0.5) (layer "B.Cu") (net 1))
 (segment (start 46.122392 92.119651) (end 46.122392 74.081726) (width 0.5) (layer "B.Cu") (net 1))
 (segment (start 73.386925 90.487817) (end 69.348772 90.487817) (width 0.5) (layer "B.Cu") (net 1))
 (segment (start 73.386925 90.487817) (end 90.58417 90.487817) (width 0.5) (layer "B.Cu") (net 1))
 (segment (start 92.969914 88.102073) (end 103.45119 88.102073) (width 0.5) (layer "B.Cu") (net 1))
 (segment (start 69.348772 90.487817) (end 68.396589 91.44) (width 0.5) (layer "B.Cu") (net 1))
 (segment (start 90.58417 90.487817) (end 92.969914 88.102073) (width 0.5) (layer "B.Cu") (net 1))
 (segment (start 46.122392 92.119651) (end 44.769931 93.472112) (width 0.5) (layer "B.Cu") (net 1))
 (segment (start 93.91225 90.377073) (end 76.493517 90.377073) (width 0.5) (layer "F.Cu") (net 3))
 (segment (start 46.227888 90.932112) (end 44.769931 90.932112) (width 0.5) (layer "F.Cu") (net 3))
 (segment (start 95.612317 88.677006) (end 93.91225 90.377073) (width 0.5) (layer "F.Cu") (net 3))
 (segment (start 49.158423 88.001577) (end 46.227888 90.932112) (width 0.5) (layer "F.Cu") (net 3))
 (segment (start 124.237006 88.677006) (end 95.612317 88.677006) (width 0.5) (layer "F.Cu") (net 3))
 (segment (start 74.118021 88.001577) (end 49.158423 88.001577) (width 0.5) (layer "F.Cu") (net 3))
 (segment (start 125.28 89.72) (end 124.237006 88.677006) (width 0.5) (layer "F.Cu") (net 3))
 (segment (start 76.493517 90.377073) (end 74.118021 88.001577) (width 0.5) (layer "F.Cu") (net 3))
 (via (at 125.28 89.72) (size 1.4) (drill 1.1) (layers "F.Cu" "B.Cu") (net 3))
 (segment (start 128.280077 92.720077) (end 130.23405 92.720077) (width 0.5) (layer "B.Cu") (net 3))
 (segment (start 149.44 92.71) (end 146.912293 90.182293) (width 0.4) (layer "B.Cu") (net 3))
 (segment (start 149.44 92.71) (end 168.326417 92.71) (width 0.4) (layer "B.Cu") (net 3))
 (segment (start 168.326417 92.71) (end 168.349289 92.732872) (width 0.4) (layer "B.Cu") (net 3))
 (segment (start 146.912293 76.100443) (end 149.337293 73.675443) (width 0.4) (layer "B.Cu") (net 3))
 (segment (start 130.23405 92.720077) (end 149.429923 92.720077) (width 0.5) (layer "B.Cu") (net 3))
 (segment (start 146.912293 90.182293) (end 146.912293 76.100443) (width 0.4) (layer "B.Cu") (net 3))
 (segment (start 125.28 89.72) (end 128.280077 92.720077) (width 0.5) (layer "B.Cu") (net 3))
 (segment (start 187.547645 95.724004) (end 177.153641 85.33) (width 0.5) (layer "F.Cu") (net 5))
 (segment (start 177.153641 85.33) (end 47.832043 85.33) (width 0.5) (layer "F.Cu") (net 5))
 (segment (start 47.832043 85.33) (end 44.769931 88.392112) (width 0.5) (layer "F.Cu") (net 5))
 (segment (start 187.547645 95.724004) (end 195.135639 88.13601) (width 0.5) (layer "B.Cu") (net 5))
 (segment (start 225.222533 90.455484) (end 238.822146 76.855871) (width 0.5) (layer "B.Cu") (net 5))
 (segment (start 238.822146 76.855871) (end 250.318013 76.855871) (width 0.5) (layer "B.Cu") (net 5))
 (segment (start 206.706408 87.036011) (end 221.80306 87.036011) (width 0.5) (layer "B.Cu") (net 5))
 (segment (start 195.135639 88.13601) (end 205.606409 88.13601) (width 0.5) (layer "B.Cu") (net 5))
 (segment (start 221.80306 87.036011) (end 225.222533 90.455484) (width 0.5) (layer "B.Cu") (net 5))
 (segment (start 205.606409 88.13601) (end 206.706408 87.036011) (width 0.5) (layer "B.Cu") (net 5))
 (segment (start 47.752112 96.012112) (end 56.077012 104.337012) (width 0.5) (layer "F.Cu") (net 14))
 (segment (start 56.077012 104.337012) (end 56.077012 108.433432) (width 0.5) (layer "F.Cu") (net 14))
 (segment (start 44.769931 96.012112) (end 47.752112 96.012112) (width 0.5) (layer "F.Cu") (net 14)))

